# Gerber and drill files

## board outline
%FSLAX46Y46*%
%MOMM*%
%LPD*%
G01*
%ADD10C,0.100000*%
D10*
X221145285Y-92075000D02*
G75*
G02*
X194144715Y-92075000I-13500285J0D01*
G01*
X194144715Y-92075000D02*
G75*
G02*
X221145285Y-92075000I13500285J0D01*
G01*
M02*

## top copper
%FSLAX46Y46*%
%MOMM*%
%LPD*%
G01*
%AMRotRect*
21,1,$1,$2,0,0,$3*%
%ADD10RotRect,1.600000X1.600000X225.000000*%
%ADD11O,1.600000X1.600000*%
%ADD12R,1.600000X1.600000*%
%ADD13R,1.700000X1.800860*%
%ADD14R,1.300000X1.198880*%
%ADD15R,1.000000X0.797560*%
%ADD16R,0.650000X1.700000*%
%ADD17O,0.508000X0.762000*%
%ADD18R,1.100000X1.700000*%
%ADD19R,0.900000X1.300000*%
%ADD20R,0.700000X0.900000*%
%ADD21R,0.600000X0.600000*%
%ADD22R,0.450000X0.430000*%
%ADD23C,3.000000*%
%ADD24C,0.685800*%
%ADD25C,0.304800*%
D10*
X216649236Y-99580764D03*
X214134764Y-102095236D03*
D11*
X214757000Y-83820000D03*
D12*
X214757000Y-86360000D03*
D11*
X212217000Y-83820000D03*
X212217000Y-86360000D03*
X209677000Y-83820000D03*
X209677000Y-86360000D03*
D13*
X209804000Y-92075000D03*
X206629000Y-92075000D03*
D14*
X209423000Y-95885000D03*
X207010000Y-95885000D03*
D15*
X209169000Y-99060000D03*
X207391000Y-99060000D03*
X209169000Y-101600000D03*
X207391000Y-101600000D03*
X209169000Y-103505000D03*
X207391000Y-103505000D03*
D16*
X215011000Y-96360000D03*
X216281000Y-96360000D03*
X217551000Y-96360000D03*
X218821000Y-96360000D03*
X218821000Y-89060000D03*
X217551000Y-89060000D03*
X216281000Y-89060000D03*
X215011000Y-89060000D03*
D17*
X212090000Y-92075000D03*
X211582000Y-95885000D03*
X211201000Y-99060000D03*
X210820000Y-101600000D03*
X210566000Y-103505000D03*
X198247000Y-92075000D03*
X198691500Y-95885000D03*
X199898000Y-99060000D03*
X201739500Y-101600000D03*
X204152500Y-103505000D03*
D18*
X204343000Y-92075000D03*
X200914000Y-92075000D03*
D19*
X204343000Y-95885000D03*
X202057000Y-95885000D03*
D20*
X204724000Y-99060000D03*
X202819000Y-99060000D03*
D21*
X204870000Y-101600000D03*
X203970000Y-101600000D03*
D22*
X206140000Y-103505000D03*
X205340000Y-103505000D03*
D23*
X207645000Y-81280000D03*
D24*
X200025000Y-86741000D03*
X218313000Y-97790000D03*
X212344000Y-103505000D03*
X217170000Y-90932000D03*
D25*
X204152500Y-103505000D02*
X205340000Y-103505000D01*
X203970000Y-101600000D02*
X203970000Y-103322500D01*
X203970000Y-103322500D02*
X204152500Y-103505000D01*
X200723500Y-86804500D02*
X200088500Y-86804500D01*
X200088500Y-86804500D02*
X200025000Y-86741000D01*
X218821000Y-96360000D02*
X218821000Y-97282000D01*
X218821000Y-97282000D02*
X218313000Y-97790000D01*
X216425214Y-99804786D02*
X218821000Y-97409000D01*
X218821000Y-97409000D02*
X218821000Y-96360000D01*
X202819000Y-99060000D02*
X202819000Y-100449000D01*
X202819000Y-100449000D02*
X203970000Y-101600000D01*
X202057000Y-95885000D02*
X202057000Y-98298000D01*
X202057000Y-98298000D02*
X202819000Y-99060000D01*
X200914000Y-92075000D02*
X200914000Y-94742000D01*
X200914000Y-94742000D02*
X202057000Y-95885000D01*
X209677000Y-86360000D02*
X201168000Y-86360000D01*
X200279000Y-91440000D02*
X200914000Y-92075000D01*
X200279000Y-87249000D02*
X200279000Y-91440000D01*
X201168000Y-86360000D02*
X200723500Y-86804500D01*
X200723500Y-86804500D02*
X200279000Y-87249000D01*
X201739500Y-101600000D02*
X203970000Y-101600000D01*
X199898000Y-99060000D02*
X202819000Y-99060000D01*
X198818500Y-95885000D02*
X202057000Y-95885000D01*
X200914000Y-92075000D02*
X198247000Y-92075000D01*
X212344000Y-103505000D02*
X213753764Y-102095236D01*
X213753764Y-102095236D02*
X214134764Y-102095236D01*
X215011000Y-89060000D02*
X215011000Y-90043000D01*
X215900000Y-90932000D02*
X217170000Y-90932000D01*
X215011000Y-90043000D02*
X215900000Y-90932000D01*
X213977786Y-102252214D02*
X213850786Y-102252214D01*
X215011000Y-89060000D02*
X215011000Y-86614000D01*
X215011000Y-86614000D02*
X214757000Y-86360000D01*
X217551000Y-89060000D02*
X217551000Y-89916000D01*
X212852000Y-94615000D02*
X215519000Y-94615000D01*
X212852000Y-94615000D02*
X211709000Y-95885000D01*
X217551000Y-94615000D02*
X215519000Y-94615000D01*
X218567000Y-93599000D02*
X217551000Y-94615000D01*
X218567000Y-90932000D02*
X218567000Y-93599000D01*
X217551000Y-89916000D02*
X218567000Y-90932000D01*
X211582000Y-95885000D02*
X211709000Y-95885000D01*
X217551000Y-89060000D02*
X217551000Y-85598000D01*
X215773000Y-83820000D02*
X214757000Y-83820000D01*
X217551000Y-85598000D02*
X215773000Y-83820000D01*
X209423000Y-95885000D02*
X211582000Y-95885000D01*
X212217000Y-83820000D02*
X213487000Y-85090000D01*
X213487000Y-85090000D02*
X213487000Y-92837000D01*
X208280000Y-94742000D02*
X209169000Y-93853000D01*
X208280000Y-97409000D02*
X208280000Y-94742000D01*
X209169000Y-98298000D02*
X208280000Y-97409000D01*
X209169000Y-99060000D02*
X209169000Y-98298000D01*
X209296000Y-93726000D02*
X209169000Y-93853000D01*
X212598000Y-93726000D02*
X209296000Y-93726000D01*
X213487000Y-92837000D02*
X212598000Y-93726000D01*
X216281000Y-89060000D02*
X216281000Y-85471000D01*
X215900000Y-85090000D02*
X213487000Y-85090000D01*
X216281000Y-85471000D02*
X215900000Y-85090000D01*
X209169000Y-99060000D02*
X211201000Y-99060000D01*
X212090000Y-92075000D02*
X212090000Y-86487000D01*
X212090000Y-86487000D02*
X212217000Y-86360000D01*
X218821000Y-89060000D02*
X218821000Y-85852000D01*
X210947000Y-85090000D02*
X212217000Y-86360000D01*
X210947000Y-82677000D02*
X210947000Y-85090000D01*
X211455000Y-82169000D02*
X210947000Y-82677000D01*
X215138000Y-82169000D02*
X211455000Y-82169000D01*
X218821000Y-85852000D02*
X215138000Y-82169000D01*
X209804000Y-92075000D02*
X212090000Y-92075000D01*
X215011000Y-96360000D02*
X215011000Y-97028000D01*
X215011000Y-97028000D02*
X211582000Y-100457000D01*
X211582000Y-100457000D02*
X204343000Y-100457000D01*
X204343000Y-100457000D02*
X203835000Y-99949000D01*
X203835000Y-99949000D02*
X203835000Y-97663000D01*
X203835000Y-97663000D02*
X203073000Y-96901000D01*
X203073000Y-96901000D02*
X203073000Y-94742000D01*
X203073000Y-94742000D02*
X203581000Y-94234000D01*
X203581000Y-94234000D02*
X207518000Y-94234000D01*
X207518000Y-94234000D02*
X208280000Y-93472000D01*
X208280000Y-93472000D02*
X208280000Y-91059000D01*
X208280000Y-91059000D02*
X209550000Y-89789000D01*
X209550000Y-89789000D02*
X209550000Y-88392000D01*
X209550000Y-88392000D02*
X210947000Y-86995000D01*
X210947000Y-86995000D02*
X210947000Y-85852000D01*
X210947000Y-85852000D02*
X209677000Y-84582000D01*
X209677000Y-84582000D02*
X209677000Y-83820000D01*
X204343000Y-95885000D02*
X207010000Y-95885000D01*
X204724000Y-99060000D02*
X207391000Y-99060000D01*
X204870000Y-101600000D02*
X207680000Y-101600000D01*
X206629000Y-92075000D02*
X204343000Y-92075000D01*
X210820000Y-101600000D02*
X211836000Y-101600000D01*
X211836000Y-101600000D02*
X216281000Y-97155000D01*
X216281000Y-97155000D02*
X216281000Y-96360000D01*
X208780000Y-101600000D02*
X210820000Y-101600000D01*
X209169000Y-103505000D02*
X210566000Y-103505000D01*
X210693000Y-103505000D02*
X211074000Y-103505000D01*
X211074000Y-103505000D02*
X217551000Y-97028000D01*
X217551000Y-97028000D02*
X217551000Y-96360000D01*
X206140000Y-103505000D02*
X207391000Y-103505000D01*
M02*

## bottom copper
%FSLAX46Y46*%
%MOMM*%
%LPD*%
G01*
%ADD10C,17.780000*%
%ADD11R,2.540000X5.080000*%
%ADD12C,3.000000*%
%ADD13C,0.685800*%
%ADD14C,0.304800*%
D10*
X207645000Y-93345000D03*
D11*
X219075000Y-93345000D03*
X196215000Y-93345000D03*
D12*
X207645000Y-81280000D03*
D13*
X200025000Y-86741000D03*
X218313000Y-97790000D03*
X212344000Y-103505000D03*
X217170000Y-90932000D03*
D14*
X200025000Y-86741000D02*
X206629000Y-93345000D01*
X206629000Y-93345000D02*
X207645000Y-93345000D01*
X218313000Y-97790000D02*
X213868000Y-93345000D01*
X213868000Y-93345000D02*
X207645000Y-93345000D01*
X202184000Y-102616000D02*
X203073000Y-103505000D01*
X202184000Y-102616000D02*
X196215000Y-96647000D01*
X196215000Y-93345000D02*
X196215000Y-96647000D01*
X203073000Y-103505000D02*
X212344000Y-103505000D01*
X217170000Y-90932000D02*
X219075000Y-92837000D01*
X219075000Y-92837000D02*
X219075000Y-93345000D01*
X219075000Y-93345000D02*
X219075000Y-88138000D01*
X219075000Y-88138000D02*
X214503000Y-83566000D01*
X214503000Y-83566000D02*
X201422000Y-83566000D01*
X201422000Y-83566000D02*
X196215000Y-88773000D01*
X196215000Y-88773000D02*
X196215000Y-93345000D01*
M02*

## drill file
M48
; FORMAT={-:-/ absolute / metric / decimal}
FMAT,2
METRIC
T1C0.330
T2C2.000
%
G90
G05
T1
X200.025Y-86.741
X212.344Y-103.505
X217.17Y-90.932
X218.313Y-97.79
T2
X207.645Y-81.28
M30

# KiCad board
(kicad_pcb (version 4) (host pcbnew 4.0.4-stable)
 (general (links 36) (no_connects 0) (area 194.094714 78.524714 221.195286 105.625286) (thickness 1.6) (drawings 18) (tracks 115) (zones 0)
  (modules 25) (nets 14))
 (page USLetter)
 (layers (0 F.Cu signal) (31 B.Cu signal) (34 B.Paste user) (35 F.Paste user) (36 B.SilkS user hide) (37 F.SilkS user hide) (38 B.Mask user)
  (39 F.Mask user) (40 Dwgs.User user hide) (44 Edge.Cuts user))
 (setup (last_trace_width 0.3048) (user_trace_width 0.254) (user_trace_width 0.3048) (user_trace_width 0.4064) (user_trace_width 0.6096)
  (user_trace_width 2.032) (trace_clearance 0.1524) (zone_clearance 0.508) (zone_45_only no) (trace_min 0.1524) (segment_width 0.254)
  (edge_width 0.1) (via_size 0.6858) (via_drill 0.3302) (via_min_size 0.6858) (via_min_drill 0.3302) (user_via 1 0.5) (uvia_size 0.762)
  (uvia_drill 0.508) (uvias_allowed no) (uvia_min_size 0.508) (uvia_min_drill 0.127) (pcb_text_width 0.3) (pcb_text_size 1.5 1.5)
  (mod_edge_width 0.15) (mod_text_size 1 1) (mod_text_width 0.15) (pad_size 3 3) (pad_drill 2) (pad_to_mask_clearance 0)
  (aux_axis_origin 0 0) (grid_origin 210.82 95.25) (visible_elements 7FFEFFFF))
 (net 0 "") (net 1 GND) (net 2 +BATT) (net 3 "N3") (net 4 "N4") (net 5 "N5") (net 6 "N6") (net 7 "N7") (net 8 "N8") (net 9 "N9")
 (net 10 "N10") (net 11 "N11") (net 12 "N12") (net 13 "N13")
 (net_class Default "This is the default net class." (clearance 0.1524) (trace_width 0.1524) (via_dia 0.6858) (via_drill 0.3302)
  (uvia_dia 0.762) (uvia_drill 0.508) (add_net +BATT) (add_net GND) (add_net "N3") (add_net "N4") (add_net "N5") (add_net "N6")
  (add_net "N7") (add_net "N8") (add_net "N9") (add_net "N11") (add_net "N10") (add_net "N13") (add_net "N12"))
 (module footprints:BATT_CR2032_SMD (layer B.Cu) (at 207.645 93.345 180)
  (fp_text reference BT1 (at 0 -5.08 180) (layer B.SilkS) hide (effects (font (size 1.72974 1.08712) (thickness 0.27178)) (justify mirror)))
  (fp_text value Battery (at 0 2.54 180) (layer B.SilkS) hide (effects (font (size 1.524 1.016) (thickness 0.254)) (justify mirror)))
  (pad 2 smd circle (at 0 0 180) (size 17.78 17.78) (layers B.Cu B.Paste B.Mask) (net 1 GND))
  (pad 1 smd rect (at -11.43 0 180) (size 2.54 5.08) (layers B.Cu B.Paste B.Mask) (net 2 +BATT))
  (pad 1 smd rect (at 11.43 0 180) (size 2.54 5.08) (layers B.Cu B.Paste B.Mask) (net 2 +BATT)))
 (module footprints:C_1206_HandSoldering (layer F.Cu) (at 215.392 100.838 225)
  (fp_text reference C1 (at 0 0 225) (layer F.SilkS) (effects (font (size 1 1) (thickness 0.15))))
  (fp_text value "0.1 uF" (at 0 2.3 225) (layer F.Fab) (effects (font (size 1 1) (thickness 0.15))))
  (pad 1 smd rect (at -1.778 0 225) (size 1.6 1.6) (layers F.Cu F.Paste F.Mask) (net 1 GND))
  (pad 2 smd rect (at 1.778 0 225) (size 1.6 1.6) (layers F.Cu F.Paste F.Mask) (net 2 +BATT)))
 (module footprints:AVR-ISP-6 (layer F.Cu) (at 214.757 83.82 270)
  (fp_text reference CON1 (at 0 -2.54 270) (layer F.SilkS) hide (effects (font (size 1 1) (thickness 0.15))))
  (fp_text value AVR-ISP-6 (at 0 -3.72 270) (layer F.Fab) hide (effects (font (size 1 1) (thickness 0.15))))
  (pad 1 smd oval (at 0 0 270) (size 1.6 1.6) (layers F.Cu F.Paste F.Mask) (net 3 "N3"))
  (pad 2 smd rect (at 2.54 0 270) (size 1.6 1.6) (layers F.Cu F.Paste F.Mask) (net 2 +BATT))
  (pad 3 smd oval (at 0 2.54 270) (size 1.6 1.6) (layers F.Cu F.Paste F.Mask) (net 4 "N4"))
  (pad 4 smd oval (at 2.54 2.54 270) (size 1.6 1.6) (layers F.Cu F.Paste F.Mask) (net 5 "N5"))
  (pad 5 smd oval (at 0 5.08 270) (size 1.6 1.6) (layers F.Cu F.Paste F.Mask) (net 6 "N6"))
  (pad 6 smd oval (at 2.54 5.08 270) (size 1.6 1.6) (layers F.Cu F.Paste F.Mask) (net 1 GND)))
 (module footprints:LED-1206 (layer F.Cu) (at 208.28 92.075)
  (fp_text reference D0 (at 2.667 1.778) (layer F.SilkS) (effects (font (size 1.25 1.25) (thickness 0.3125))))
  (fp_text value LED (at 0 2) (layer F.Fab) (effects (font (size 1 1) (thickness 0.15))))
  (pad 2 smd rect (at 1.524 0 180) (size 1.7 1.80086) (layers F.Cu F.Paste F.Mask) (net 5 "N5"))
  (pad 1 smd rect (at -1.651 0 180) (size 1.7 1.80086) (layers F.Cu F.Paste F.Mask) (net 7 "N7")))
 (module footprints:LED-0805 (layer F.Cu) (at 208.28 95.885)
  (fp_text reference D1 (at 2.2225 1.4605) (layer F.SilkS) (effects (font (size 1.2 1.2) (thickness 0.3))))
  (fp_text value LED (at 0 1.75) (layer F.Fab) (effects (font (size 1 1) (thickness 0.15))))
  (pad 2 smd rect (at 1.143 0 180) (size 1.3 1.19888) (layers F.Cu F.Paste F.Mask) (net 3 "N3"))
  (pad 1 smd rect (at -1.27 0 180) (size 1.3 1.19888) (layers F.Cu F.Paste F.Mask) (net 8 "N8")))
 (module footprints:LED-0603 (layer F.Cu) (at 208.28 99.06)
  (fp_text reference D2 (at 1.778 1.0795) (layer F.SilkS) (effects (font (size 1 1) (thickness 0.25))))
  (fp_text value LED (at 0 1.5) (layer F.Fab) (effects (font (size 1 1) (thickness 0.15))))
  (pad 2 smd rect (at 0.889 0 180) (size 1 0.79756) (layers F.Cu F.Paste F.Mask) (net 4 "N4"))
  (pad 1 smd rect (at -0.889 0 180) (size 1 0.79756) (layers F.Cu F.Paste F.Mask) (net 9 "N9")))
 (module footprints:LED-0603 (layer F.Cu) (at 208.28 101.6)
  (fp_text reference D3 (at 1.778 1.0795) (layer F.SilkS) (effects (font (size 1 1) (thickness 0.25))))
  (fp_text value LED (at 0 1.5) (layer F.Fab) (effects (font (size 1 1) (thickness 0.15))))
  (pad 2 smd rect (at 0.889 0 180) (size 1 0.79756) (layers F.Cu F.Paste F.Mask) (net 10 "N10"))
  (pad 1 smd rect (at -0.889 0 180) (size 1 0.79756) (layers F.Cu F.Paste F.Mask) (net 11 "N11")))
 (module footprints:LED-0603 (layer F.Cu) (at 208.28 103.505)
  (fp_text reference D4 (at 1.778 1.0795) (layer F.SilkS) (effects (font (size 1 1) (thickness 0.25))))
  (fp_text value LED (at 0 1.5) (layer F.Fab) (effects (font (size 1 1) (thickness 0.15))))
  (pad 2 smd rect (at 0.889 0 180) (size 1 0.79756) (layers F.Cu F.Paste F.Mask) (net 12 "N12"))
  (pad 1 smd rect (at -0.889 0 180) (size 1 0.79756) (layers F.Cu F.Paste F.Mask) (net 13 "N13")))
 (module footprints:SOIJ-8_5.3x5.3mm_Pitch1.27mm (layer F.Cu) (at 216.916 92.71 90)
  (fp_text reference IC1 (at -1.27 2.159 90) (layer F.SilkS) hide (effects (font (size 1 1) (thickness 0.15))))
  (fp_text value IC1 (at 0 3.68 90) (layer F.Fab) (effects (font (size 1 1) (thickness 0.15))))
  (pad 1 smd rect (at -3.65 -1.905 90) (size 1.7 0.65) (layers F.Cu F.Paste F.Mask) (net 6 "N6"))
  (pad 2 smd rect (at -3.65 -0.635 90) (size 1.7 0.65) (layers F.Cu F.Paste F.Mask) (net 10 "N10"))
  (pad 3 smd rect (at -3.65 0.635 90) (size 1.7 0.65) (layers F.Cu F.Paste F.Mask) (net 12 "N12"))
  (pad 4 smd rect (at -3.65 1.905 90) (size 1.7 0.65) (layers F.Cu F.Paste F.Mask) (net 1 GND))
  (pad 5 smd rect (at 3.65 1.905 90) (size 1.7 0.65) (layers F.Cu F.Paste F.Mask) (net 5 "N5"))
  (pad 6 smd rect (at 3.65 0.635 90) (size 1.7 0.65) (layers F.Cu F.Paste F.Mask) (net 3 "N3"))
  (pad 7 smd rect (at 3.65 -0.635 90) (size 1.7 0.65) (layers F.Cu F.Paste F.Mask) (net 4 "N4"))
  (pad 8 smd rect (at 3.65 -1.905 90) (size 1.7 0.65) (layers F.Cu F.Paste F.Mask) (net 2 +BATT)))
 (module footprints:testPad (layer F.Cu) (at 212.09 92.075)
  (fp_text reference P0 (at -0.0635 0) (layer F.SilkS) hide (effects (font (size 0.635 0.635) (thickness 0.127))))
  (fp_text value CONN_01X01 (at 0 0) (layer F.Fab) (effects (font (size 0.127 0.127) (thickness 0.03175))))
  (pad 1 smd oval (at 0 0) (size 0.508 0.762) (layers F.Cu F.Paste F.Mask) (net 5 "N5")))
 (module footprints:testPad (layer F.Cu) (at 211.582 95.885)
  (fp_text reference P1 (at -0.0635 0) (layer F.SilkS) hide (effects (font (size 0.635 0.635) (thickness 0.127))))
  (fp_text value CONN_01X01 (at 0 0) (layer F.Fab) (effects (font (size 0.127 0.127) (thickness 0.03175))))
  (pad 1 smd oval (at 0 0) (size 0.508 0.762) (layers F.Cu F.Paste F.Mask) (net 3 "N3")))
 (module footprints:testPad (layer F.Cu) (at 211.201 99.06)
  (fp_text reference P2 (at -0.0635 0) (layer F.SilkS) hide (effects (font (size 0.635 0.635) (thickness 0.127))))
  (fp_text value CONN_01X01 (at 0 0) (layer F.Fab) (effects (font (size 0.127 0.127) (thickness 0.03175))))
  (pad 1 smd oval (at 0 0) (size 0.508 0.762) (layers F.Cu F.Paste F.Mask) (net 4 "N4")))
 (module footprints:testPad (layer F.Cu) (at 210.82 101.6)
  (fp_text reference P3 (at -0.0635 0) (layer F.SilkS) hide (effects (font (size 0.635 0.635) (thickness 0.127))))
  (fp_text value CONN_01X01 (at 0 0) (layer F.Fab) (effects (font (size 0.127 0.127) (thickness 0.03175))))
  (pad 1 smd oval (at 0 0) (size 0.508 0.762) (layers F.Cu F.Paste F.Mask) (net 10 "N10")))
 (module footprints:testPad (layer F.Cu) (at 210.566 103.505)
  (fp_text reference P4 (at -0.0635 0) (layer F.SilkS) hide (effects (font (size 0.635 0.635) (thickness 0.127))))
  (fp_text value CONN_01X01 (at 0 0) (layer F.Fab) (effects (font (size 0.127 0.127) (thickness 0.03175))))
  (pad 1 smd oval (at 0 0) (size 0.508 0.762) (layers F.Cu F.Paste F.Mask) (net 12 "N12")))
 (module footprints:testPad (layer F.Cu) (at 198.247 92.075)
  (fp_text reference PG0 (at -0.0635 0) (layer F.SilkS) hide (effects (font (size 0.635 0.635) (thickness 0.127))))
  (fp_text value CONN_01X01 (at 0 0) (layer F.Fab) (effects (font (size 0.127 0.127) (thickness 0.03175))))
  (pad 1 smd oval (at 0 0) (size 0.508 0.762) (layers F.Cu F.Paste F.Mask) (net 1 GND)))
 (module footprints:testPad (layer F.Cu) (at 198.6915 95.885)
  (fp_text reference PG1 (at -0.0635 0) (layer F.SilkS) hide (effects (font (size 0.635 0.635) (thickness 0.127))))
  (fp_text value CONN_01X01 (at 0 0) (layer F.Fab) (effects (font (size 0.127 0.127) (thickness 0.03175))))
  (pad 1 smd oval (at 0 0) (size 0.508 0.762) (layers F.Cu F.Paste F.Mask) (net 1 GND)))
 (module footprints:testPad (layer F.Cu) (at 199.898 99.06)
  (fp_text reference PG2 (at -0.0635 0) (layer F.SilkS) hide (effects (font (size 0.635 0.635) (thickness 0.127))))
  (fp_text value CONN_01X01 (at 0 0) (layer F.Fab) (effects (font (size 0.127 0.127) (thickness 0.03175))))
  (pad 1 smd oval (at 0 0) (size 0.508 0.762) (layers F.Cu F.Paste F.Mask) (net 1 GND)))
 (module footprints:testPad (layer F.Cu) (at 201.7395 101.6)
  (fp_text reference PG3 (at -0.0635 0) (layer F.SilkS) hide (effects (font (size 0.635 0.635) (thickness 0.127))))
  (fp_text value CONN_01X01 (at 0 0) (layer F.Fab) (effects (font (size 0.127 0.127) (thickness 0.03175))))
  (pad 1 smd oval (at 0 0) (size 0.508 0.762) (layers F.Cu F.Paste F.Mask) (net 1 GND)))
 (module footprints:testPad (layer F.Cu) (at 204.1525 103.505)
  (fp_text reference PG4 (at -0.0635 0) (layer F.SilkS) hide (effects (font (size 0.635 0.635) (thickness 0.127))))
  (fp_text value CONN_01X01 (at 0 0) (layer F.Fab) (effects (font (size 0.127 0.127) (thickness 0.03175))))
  (pad 1 smd oval (at 0 0) (size 0.508 0.762) (layers F.Cu F.Paste F.Mask) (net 1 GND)))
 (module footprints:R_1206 (layer F.Cu) (at 202.565 92.075 180)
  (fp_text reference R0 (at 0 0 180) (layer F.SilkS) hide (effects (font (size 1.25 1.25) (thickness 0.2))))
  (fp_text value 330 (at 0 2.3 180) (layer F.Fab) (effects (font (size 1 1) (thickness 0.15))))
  (pad 1 smd rect (at -1.778 0 180) (size 1.1 1.7) (layers F.Cu F.Paste F.Mask) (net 7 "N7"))
  (pad 2 smd rect (at 1.651 0 180) (size 1.1 1.7) (layers F.Cu F.Paste F.Mask) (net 1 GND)))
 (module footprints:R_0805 (layer F.Cu) (at 203.2 95.885 180)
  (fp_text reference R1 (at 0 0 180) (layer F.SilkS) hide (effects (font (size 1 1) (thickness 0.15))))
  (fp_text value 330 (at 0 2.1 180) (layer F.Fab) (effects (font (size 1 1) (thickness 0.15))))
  (pad 1 smd rect (at -1.143 0 180) (size 0.9 1.3) (layers F.Cu F.Paste F.Mask) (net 8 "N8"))
  (pad 2 smd rect (at 1.143 0 180) (size 0.9 1.3) (layers F.Cu F.Paste F.Mask) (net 1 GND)))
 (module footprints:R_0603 (layer F.Cu) (at 203.835 99.06 180)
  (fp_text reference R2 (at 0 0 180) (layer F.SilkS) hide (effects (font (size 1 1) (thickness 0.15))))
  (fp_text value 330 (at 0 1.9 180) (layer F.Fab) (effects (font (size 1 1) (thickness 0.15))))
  (pad 1 smd rect (at -0.889 0 180) (size 0.7 0.9) (layers F.Cu F.Paste F.Mask) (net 9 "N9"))
  (pad 2 smd rect (at 1.016 0 180) (size 0.7 0.9) (layers F.Cu F.Paste F.Mask) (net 1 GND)))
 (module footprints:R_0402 (layer F.Cu) (at 204.47 101.6 180)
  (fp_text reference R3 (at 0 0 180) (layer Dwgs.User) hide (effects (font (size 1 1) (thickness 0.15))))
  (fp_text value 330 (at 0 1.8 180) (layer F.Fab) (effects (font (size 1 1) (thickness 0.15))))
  (pad 1 smd rect (at -0.4 0 180) (size 0.6 0.6) (layers F.Cu F.Paste F.Mask) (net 11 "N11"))
  (pad 2 smd rect (at 0.5 0 180) (size 0.6 0.6) (layers F.Cu F.Paste F.Mask) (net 1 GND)))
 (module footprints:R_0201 (layer F.Cu) (at 205.74 103.505 180)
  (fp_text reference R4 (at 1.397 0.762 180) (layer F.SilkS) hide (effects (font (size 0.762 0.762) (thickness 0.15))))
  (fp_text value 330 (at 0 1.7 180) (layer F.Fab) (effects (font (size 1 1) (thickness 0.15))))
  (pad 1 smd rect (at -0.4 0 180) (size 0.45 0.43) (layers F.Cu F.Paste F.Mask) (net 13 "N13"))
  (pad 2 smd rect (at 0.4 0 180) (size 0.45 0.43) (layers F.Cu F.Paste F.Mask) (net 1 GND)))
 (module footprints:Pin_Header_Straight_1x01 (layer F.Cu) (at 207.645 81.28)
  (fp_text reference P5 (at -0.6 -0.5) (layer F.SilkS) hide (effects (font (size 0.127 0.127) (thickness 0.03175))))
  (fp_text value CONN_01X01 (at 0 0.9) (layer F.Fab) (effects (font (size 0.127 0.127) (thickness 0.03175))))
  (pad 1 thru_hole circle (at 0 0) (size 3 3) (drill 2) (layers *.Cu *.Mask)))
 (gr_circle (center 207.645 92.075) (end 197.485 83.185) (layer Edge.Cuts) (width 0.1))
 (segment (start 204.1525 103.505) (end 205.34 103.505) (width 0.3048) (layer F.Cu) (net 1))
 (segment (start 203.97 101.6) (end 203.97 103.3225) (width 0.3048) (layer F.Cu) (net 1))
 (segment (start 203.97 103.3225) (end 204.1525 103.505) (width 0.3048) (layer F.Cu) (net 1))
 (segment (start 200.7235 86.8045) (end 200.0885 86.8045) (width 0.3048) (layer F.Cu) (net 1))
 (segment (start 200.025 86.741) (end 206.629 93.345) (width 0.3048) (layer B.Cu) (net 1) (status 20))
 (via (at 200.025 86.741) (size 0.6858) (drill 0.3302) (layers F.Cu B.Cu) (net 1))
 (segment (start 200.0885 86.8045) (end 200.025 86.741) (width 0.3048) (layer F.Cu) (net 1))
 (segment (start 206.629 93.345) (end 207.645 93.345) (width 0.3048) (layer B.Cu) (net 1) (status 30))
 (segment (start 218.821 96.36) (end 218.821 97.282) (width 0.3048) (layer F.Cu) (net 1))
 (segment (start 218.313 97.79) (end 213.868 93.345) (width 0.3048) (layer B.Cu) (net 1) (status 20))
 (via (at 218.313 97.79) (size 0.6858) (drill 0.3302) (layers F.Cu B.Cu) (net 1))
 (segment (start 218.821 97.282) (end 218.313 97.79) (width 0.3048) (layer F.Cu) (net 1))
 (segment (start 213.868 93.345) (end 207.645 93.345) (width 0.3048) (layer B.Cu) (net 1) (status 30))
 (segment (start 216.425214 99.804786) (end 218.821 97.409) (width 0.3048) (layer F.Cu) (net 1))
 (segment (start 218.821 97.409) (end 218.821 96.36) (width 0.3048) (layer F.Cu) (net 1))
 (segment (start 202.819 99.06) (end 202.819 100.449) (width 0.3048) (layer F.Cu) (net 1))
 (segment (start 202.819 100.449) (end 203.97 101.6) (width 0.3048) (layer F.Cu) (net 1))
 (segment (start 202.057 95.885) (end 202.057 98.298) (width 0.3048) (layer F.Cu) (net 1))
 (segment (start 202.057 98.298) (end 202.819 99.06) (width 0.3048) (layer F.Cu) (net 1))
 (segment (start 200.914 92.075) (end 200.914 94.742) (width 0.3048) (layer F.Cu) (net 1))
 (segment (start 200.914 94.742) (end 202.057 95.885) (width 0.3048) (layer F.Cu) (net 1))
 (segment (start 209.677 86.36) (end 201.168 86.36) (width 0.3048) (layer F.Cu) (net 1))
 (segment (start 200.279 91.44) (end 200.914 92.075) (width 0.3048) (layer F.Cu) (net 1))
 (segment (start 200.279 87.249) (end 200.279 91.44) (width 0.3048) (layer F.Cu) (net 1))
 (segment (start 201.168 86.36) (end 200.7235 86.8045) (width 0.3048) (layer F.Cu) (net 1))
 (segment (start 200.7235 86.8045) (end 200.279 87.249) (width 0.3048) (layer F.Cu) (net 1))
 (segment (start 201.7395 101.6) (end 203.97 101.6) (width 0.3048) (layer F.Cu) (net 1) (status 10))
 (segment (start 199.898 99.06) (end 202.819 99.06) (width 0.3048) (layer F.Cu) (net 1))
 (segment (start 198.8185 95.885) (end 202.057 95.885) (width 0.3048) (layer F.Cu) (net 1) (status 10))
 (segment (start 200.914 92.075) (end 198.247 92.075) (width 0.3048) (layer F.Cu) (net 1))
 (segment (start 202.184 102.616) (end 203.073 103.505) (width 0.3048) (layer B.Cu) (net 2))
 (segment (start 202.184 102.616) (end 196.215 96.647) (width 0.3048) (layer B.Cu) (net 2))
 (segment (start 196.215 93.345) (end 196.215 96.647) (width 0.3048) (layer B.Cu) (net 2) (status 10))
 (segment (start 212.344 103.505) (end 213.753764 102.095236) (width 0.3048) (layer F.Cu) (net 2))
 (via (at 212.344 103.505) (size 0.6858) (drill 0.3302) (layers F.Cu B.Cu) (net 2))
 (segment (start 203.073 103.505) (end 212.344 103.505) (width 0.3048) (layer B.Cu) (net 2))
 (segment (start 213.753764 102.095236) (end 214.134764 102.095236) (width 0.3048) (layer F.Cu) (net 2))
 (segment (start 215.011 89.06) (end 215.011 90.043) (width 0.3048) (layer F.Cu) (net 2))
 (segment (start 217.17 90.932) (end 219.075 92.837) (width 0.3048) (layer B.Cu) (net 2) (status 20))
 (via (at 217.17 90.932) (size 0.6858) (drill 0.3302) (layers F.Cu B.Cu) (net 2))
 (segment (start 215.9 90.932) (end 217.17 90.932) (width 0.3048) (layer F.Cu) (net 2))
 (segment (start 215.011 90.043) (end 215.9 90.932) (width 0.3048) (layer F.Cu) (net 2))
 (segment (start 219.075 92.837) (end 219.075 93.345) (width 0.3048) (layer B.Cu) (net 2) (status 30))
 (segment (start 219.075 93.345) (end 219.075 88.138) (width 0.3048) (layer B.Cu) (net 2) (status 10))
 (segment (start 219.075 88.138) (end 214.503 83.566) (width 0.3048) (layer B.Cu) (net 2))
 (segment (start 214.503 83.566) (end 201.422 83.566) (width 0.3048) (layer B.Cu) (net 2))
 (segment (start 201.422 83.566) (end 196.215 88.773) (width 0.3048) (layer B.Cu) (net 2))
 (segment (start 196.215 88.773) (end 196.215 93.345) (width 0.3048) (layer B.Cu) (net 2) (status 20))
 (segment (start 213.977786 102.252214) (end 213.850786 102.252214) (width 0.3048) (layer F.Cu) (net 2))
 (segment (start 215.011 89.06) (end 215.011 86.614) (width 0.3048) (layer F.Cu) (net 2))
 (segment (start 215.011 86.614) (end 214.757 86.36) (width 0.3048) (layer F.Cu) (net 2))
 (segment (start 217.551 89.06) (end 217.551 89.916) (width 0.3048) (layer F.Cu) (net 3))
 (segment (start 212.852 94.615) (end 215.519 94.615) (width 0.3048) (layer F.Cu) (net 3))
 (segment (start 212.852 94.615) (end 211.709 95.885) (width 0.3048) (layer F.Cu) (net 3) (status 20))
 (segment (start 217.551 94.615) (end 215.519 94.615) (width 0.3048) (layer F.Cu) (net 3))
 (segment (start 218.567 93.599) (end 217.551 94.615) (width 0.3048) (layer F.Cu) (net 3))
 (segment (start 218.567 90.932) (end 218.567 93.599) (width 0.3048) (layer F.Cu) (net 3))
 (segment (start 217.551 89.916) (end 218.567 90.932) (width 0.3048) (layer F.Cu) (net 3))
 (segment (start 211.582 95.885) (end 211.709 95.885) (width 0.3048) (layer F.Cu) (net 3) (status 30))
 (segment (start 217.551 89.06) (end 217.551 85.598) (width 0.3048) (layer F.Cu) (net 3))
 (segment (start 215.773 83.82) (end 214.757 83.82) (width 0.3048) (layer F.Cu) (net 3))
 (segment (start 217.551 85.598) (end 215.773 83.82) (width 0.3048) (layer F.Cu) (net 3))
 (segment (start 209.423 95.885) (end 211.582 95.885) (width 0.3048) (layer F.Cu) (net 3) (status 20))
 (segment (start 212.217 83.82) (end 213.487 85.09) (width 0.3048) (layer F.Cu) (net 4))
 (segment (start 213.487 85.09) (end 213.487 92.837) (width 0.3048) (layer F.Cu) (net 4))
 (segment (start 208.28 94.742) (end 209.169 93.853) (width 0.3048) (layer F.Cu) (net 4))
 (segment (start 208.28 97.409) (end 208.28 94.742) (width 0.3048) (layer F.Cu) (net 4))
 (segment (start 209.169 98.298) (end 208.28 97.409) (width 0.3048) (layer F.Cu) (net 4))
 (segment (start 209.169 99.06) (end 209.169 98.298) (width 0.3048) (layer F.Cu) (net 4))
 (segment (start 209.296 93.726) (end 209.169 93.853) (width 0.3048) (layer F.Cu) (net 4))
 (segment (start 212.598 93.726) (end 209.296 93.726) (width 0.3048) (layer F.Cu) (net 4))
 (segment (start 213.487 92.837) (end 212.598 93.726) (width 0.3048) (layer F.Cu) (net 4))
 (segment (start 216.281 89.06) (end 216.281 85.471) (width 0.3048) (layer F.Cu) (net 4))
 (segment (start 215.9 85.09) (end 213.487 85.09) (width 0.3048) (layer F.Cu) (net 4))
 (segment (start 216.281 85.471) (end 215.9 85.09) (width 0.3048) (layer F.Cu) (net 4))
 (segment (start 209.169 99.06) (end 211.201 99.06) (width 0.3048) (layer F.Cu) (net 4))
 (segment (start 212.09 92.075) (end 212.09 86.487) (width 0.3048) (layer F.Cu) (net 5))
 (segment (start 212.09 86.487) (end 212.217 86.36) (width 0.3048) (layer F.Cu) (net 5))
 (segment (start 218.821 89.06) (end 218.821 85.852) (width 0.3048) (layer F.Cu) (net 5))
 (segment (start 210.947 85.09) (end 212.217 86.36) (width 0.3048) (layer F.Cu) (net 5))
 (segment (start 210.947 82.677) (end 210.947 85.09) (width 0.3048) (layer F.Cu) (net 5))
 (segment (start 211.455 82.169) (end 210.947 82.677) (width 0.3048) (layer F.Cu) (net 5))
 (segment (start 215.138 82.169) (end 211.455 82.169) (width 0.3048) (layer F.Cu) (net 5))
 (segment (start 218.821 85.852) (end 215.138 82.169) (width 0.3048) (layer F.Cu) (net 5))
 (segment (start 209.804 92.075) (end 212.09 92.075) (width 0.3048) (layer F.Cu) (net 5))
 (segment (start 215.011 96.36) (end 215.011 97.028) (width 0.3048) (layer F.Cu) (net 6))
 (segment (start 215.011 97.028) (end 211.582 100.457) (width 0.3048) (layer F.Cu) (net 6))
 (segment (start 211.582 100.457) (end 204.343 100.457) (width 0.3048) (layer F.Cu) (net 6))
 (segment (start 204.343 100.457) (end 203.835 99.949) (width 0.3048) (layer F.Cu) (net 6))
 (segment (start 203.835 99.949) (end 203.835 97.663) (width 0.3048) (layer F.Cu) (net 6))
 (segment (start 203.835 97.663) (end 203.073 96.901) (width 0.3048) (layer F.Cu) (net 6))
 (segment (start 203.073 96.901) (end 203.073 94.742) (width 0.3048) (layer F.Cu) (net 6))
 (segment (start 203.073 94.742) (end 203.581 94.234) (width 0.3048) (layer F.Cu) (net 6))
 (segment (start 203.581 94.234) (end 207.518 94.234) (width 0.3048) (layer F.Cu) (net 6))
 (segment (start 207.518 94.234) (end 208.28 93.472) (width 0.3048) (layer F.Cu) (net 6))
 (segment (start 208.28 93.472) (end 208.28 91.059) (width 0.3048) (layer F.Cu) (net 6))
 (segment (start 208.28 91.059) (end 209.55 89.789) (width 0.3048) (layer F.Cu) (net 6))
 (segment (start 209.55 89.789) (end 209.55 88.392) (width 0.3048) (layer F.Cu) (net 6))
 (segment (start 209.55 88.392) (end 210.947 86.995) (width 0.3048) (layer F.Cu) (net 6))
 (segment (start 210.947 86.995) (end 210.947 85.852) (width 0.3048) (layer F.Cu) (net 6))
 (segment (start 210.947 85.852) (end 209.677 84.582) (width 0.3048) (layer F.Cu) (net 6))
 (segment (start 209.677 84.582) (end 209.677 83.82) (width 0.3048) (layer F.Cu) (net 6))
 (segment (start 204.343 95.885) (end 207.01 95.885) (width 0.3048) (layer F.Cu) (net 8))
 (segment (start 204.724 99.06) (end 207.391 99.06) (width 0.3048) (layer F.Cu) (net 9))
 (segment (start 204.87 101.6) (end 207.68 101.6) (width 0.3048) (layer F.Cu) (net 11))
 (segment (start 206.629 92.075) (end 204.343 92.075) (width 0.3048) (layer F.Cu) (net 7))
 (segment (start 210.82 101.6) (end 211.836 101.6) (width 0.3048) (layer F.Cu) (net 10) (status 10))
 (segment (start 211.836 101.6) (end 216.281 97.155) (width 0.3048) (layer F.Cu) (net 10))
 (segment (start 216.281 97.155) (end 216.281 96.36) (width 0.3048) (layer F.Cu) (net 10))
 (segment (start 208.78 101.6) (end 210.82 101.6) (width 0.3048) (layer F.Cu) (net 10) (status 20))
 (segment (start 209.169 103.505) (end 210.566 103.505) (width 0.3048) (layer F.Cu) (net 12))
 (segment (start 210.693 103.505) (end 211.074 103.505) (width 0.3048) (layer F.Cu) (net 12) (status 10))
 (segment (start 211.074 103.505) (end 217.551 97.028) (width 0.3048) (layer F.Cu) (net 12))
 (segment (start 217.551 97.028) (end 217.551 96.36) (width 0.3048) (layer F.Cu) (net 12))
 (segment (start 206.14 103.505) (end 207.391 103.505) (width 0.3048) (layer F.Cu) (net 13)))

